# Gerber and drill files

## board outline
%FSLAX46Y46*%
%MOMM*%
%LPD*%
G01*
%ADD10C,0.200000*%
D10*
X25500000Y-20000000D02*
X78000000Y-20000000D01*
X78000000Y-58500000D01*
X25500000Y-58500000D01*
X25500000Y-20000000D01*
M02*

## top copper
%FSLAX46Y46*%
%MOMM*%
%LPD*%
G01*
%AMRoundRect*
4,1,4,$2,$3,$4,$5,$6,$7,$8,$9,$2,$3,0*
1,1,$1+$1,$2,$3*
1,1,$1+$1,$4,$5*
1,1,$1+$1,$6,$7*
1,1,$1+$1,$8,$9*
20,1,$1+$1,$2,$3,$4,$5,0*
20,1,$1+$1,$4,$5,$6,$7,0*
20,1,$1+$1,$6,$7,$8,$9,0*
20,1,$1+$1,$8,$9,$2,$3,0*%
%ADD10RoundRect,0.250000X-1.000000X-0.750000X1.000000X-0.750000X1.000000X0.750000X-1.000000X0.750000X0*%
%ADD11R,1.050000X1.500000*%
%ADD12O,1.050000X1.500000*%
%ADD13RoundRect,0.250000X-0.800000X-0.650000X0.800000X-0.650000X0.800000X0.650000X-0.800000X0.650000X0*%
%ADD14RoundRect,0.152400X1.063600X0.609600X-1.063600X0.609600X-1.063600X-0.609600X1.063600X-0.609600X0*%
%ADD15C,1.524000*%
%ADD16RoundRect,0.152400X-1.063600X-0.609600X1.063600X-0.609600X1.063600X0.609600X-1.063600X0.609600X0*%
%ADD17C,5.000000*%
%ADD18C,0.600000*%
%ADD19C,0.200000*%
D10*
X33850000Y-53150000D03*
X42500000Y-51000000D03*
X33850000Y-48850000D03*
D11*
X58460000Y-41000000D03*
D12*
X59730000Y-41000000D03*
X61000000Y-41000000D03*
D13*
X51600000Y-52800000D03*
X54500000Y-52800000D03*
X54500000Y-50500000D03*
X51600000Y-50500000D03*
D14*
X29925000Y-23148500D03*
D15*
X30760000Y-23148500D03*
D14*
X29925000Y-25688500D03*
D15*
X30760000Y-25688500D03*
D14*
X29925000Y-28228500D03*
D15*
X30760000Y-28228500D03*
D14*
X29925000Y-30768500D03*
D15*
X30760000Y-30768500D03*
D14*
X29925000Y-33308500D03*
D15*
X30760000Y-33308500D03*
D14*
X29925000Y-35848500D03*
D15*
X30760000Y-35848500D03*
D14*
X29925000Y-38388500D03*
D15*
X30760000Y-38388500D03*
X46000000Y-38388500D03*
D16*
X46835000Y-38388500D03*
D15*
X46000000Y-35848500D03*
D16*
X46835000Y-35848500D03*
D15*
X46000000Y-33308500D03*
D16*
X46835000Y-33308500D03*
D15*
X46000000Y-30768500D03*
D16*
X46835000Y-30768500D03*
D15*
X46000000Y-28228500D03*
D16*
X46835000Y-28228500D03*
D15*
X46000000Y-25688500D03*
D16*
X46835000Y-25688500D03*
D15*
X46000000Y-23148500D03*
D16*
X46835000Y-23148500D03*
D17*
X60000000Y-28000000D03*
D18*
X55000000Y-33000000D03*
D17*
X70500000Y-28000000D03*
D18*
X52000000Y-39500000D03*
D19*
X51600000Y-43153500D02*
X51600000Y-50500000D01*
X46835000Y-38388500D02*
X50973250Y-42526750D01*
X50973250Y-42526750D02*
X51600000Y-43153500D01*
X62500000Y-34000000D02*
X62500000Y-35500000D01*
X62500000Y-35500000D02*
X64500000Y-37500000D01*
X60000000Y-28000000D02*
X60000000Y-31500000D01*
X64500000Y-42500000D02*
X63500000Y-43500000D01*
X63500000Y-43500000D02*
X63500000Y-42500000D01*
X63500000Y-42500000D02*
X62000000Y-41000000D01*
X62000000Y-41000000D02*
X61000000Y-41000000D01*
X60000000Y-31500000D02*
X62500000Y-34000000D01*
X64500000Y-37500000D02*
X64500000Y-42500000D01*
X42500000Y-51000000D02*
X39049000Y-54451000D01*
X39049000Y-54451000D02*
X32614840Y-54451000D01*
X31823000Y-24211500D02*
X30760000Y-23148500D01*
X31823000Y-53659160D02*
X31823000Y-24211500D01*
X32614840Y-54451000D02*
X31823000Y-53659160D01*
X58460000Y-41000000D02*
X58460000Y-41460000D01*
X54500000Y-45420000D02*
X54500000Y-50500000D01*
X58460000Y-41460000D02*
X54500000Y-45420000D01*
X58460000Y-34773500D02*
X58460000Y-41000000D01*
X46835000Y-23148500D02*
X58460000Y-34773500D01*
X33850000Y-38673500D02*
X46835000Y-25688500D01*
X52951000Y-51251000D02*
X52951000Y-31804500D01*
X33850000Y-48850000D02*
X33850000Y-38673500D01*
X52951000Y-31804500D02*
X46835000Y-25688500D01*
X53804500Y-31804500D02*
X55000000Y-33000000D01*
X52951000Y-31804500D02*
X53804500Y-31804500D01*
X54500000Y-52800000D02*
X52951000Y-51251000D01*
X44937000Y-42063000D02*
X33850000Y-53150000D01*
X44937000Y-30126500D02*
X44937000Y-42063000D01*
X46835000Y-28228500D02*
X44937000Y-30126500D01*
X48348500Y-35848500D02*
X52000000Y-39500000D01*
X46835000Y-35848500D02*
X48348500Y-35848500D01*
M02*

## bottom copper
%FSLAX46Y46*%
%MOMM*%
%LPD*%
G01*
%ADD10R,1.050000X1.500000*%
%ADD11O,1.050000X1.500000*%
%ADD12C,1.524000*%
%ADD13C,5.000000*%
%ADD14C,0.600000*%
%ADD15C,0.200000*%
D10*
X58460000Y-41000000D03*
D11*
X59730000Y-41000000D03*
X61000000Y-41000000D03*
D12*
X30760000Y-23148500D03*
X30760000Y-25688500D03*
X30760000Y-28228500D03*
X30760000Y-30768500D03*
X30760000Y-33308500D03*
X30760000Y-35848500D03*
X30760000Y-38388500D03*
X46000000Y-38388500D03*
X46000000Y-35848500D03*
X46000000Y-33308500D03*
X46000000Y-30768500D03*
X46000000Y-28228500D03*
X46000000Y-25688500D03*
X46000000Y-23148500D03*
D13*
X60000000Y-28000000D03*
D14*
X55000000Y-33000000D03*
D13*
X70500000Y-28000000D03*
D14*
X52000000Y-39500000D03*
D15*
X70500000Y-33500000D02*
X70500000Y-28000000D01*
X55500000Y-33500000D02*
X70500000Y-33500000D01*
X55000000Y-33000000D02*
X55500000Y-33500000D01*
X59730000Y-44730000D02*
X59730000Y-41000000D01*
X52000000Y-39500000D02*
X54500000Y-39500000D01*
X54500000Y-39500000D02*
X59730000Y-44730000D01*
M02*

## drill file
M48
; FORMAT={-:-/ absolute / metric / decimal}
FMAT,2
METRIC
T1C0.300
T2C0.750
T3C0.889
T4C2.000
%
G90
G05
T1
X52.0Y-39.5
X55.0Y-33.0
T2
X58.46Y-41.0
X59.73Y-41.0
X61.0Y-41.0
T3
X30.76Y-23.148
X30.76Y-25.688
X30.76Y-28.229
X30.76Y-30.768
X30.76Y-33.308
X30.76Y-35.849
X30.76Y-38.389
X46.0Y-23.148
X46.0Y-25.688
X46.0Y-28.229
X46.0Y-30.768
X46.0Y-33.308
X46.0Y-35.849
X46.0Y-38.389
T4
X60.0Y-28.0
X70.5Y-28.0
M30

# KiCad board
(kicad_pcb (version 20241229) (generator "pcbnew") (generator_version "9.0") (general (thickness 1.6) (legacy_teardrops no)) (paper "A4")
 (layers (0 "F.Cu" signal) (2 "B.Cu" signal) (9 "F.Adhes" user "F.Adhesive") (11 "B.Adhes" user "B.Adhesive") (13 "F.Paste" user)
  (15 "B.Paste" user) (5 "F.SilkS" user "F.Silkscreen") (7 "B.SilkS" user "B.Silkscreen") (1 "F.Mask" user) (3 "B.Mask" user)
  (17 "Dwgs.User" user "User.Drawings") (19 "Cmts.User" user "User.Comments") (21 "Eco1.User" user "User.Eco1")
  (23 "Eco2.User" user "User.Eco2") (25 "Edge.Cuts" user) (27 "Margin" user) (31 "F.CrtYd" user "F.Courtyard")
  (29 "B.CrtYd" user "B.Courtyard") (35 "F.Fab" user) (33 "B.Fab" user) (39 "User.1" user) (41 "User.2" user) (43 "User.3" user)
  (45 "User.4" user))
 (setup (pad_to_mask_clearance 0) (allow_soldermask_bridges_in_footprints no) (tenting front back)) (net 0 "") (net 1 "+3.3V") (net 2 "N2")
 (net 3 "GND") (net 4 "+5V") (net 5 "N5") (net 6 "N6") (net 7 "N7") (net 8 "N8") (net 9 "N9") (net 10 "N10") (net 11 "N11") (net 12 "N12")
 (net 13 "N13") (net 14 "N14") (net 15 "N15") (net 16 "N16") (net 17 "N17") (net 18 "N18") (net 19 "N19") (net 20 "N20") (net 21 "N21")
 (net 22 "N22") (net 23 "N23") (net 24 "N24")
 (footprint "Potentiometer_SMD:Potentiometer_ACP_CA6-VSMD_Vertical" (layer "F.Cu") (at 38.175 51)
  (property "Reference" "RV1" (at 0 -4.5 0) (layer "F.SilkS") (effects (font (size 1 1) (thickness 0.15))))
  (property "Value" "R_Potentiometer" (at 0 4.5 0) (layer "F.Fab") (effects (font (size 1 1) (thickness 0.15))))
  (pad "1" smd roundrect (at -4.325 2.15) (size 2.5 2) (layers "F.Cu" "F.Mask" "F.Paste") (roundrect_rratio 0.125) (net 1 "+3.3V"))
  (pad "2" smd roundrect (at 4.325 0) (size 2.5 2) (layers "F.Cu" "F.Mask" "F.Paste") (roundrect_rratio 0.125) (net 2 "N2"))
  (pad "3" smd roundrect (at -4.325 -2.15) (size 2.5 2) (layers "F.Cu" "F.Mask" "F.Paste") (roundrect_rratio 0.125) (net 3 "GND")))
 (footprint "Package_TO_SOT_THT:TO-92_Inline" (layer "F.Cu") (at 58.46 41)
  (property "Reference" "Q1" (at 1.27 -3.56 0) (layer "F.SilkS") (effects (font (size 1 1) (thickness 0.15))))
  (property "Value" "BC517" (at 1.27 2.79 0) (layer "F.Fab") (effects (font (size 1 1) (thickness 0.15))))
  (pad "1" thru_hole rect (at 0 0) (size 1.05 1.5) (drill 0.75) (layers "*.Cu" "*.Mask") (remove_unused_layers no) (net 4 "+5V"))
  (pad "2" thru_hole oval (at 1.27 0) (size 1.05 1.5) (drill 0.75) (layers "*.Cu" "*.Mask") (remove_unused_layers no) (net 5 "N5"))
  (pad "3" thru_hole oval (at 2.54 0) (size 1.05 1.5) (drill 0.75) (layers "*.Cu" "*.Mask") (remove_unused_layers no) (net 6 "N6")))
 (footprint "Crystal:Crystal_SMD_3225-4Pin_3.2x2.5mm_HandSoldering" (layer "F.Cu") (at 53.05 51.65)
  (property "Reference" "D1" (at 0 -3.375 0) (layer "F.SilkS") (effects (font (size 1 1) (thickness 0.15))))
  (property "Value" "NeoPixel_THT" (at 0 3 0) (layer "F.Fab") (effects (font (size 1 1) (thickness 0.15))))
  (pad "1" smd roundrect (at -1.45 1.15) (size 2.1 1.8) (layers "F.Cu" "F.Mask" "F.Paste") (roundrect_rratio 0.138889) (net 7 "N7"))
  (pad "2" smd roundrect (at 1.45 1.15) (size 2.1 1.8) (layers "F.Cu" "F.Mask" "F.Paste") (roundrect_rratio 0.138889) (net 3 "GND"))
  (pad "3" smd roundrect (at 1.45 -1.15) (size 2.1 1.8) (layers "F.Cu" "F.Mask" "F.Paste") (roundrect_rratio 0.138889) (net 4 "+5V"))
  (pad "4" smd roundrect (at -1.45 -1.15) (size 2.1 1.8) (layers "F.Cu" "F.Mask" "F.Paste") (roundrect_rratio 0.138889) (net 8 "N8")))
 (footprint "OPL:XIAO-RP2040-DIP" (layer "F.Cu") (at 38.38 30.7685)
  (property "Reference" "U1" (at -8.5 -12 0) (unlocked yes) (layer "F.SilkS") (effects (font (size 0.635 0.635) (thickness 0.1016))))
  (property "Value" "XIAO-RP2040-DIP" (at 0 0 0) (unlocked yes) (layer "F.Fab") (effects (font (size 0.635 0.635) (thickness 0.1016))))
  (pad "1" smd roundrect (at -8.455 -7.62 180) (size 2.432 1.524) (layers "F.Cu" "F.Mask") (roundrect_rratio 0.1) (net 2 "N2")
   (thermal_bridge_angle 45))
  (pad "1" thru_hole circle (at -7.62 -7.62 180) (size 1.524 1.524) (drill 0.889) (layers "*.Cu" "*.Mask") (remove_unused_layers no)
   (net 2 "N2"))
  (pad "2" smd roundrect (at -8.455 -5.08 180) (size 2.432 1.524) (layers "F.Cu" "F.Mask") (roundrect_rratio 0.1) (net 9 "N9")
   (thermal_bridge_angle 45))
  (pad "2" thru_hole circle (at -7.62 -5.08 180) (size 1.524 1.524) (drill 0.889) (layers "*.Cu" "*.Mask") (remove_unused_layers no)
   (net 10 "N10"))
  (pad "3" smd roundrect (at -8.455 -2.54 180) (size 2.432 1.524) (layers "F.Cu" "F.Mask") (roundrect_rratio 0.1) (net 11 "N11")
   (thermal_bridge_angle 45))
  (pad "3" thru_hole circle (at -7.62 -2.54 180) (size 1.524 1.524) (drill 0.889) (layers "*.Cu" "*.Mask") (remove_unused_layers no)
   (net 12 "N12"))
  (pad "4" smd roundrect (at -8.455 0 180) (size 2.432 1.524) (layers "F.Cu" "F.Mask") (roundrect_rratio 0.1) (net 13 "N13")
   (thermal_bridge_angle 45))
  (pad "4" thru_hole circle (at -7.62 0 180) (size 1.524 1.524) (drill 0.889) (layers "*.Cu" "*.Mask") (remove_unused_layers no)
   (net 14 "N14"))
  (pad "5" smd roundrect (at -8.455 2.54 180) (size 2.432 1.524) (layers "F.Cu" "F.Mask") (roundrect_rratio 0.1) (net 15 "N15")
   (thermal_bridge_angle 45))
  (pad "5" thru_hole circle (at -7.62 2.54 180) (size 1.524 1.524) (drill 0.889) (layers "*.Cu" "*.Mask") (remove_unused_layers no)
   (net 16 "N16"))
  (pad "6" smd roundrect (at -8.455 5.08 180) (size 2.432 1.524) (layers "F.Cu" "F.Mask") (roundrect_rratio 0.1) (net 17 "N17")
   (thermal_bridge_angle 45))
  (pad "6" thru_hole circle (at -7.62 5.08 180) (size 1.524 1.524) (drill 0.889) (layers "*.Cu" "*.Mask") (remove_unused_layers no)
   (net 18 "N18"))
  (pad "7" smd roundrect (at -8.455 7.62 180) (size 2.432 1.524) (layers "F.Cu" "F.Mask") (roundrect_rratio 0.1) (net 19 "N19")
   (thermal_bridge_angle 45))
  (pad "7" thru_hole circle (at -7.62 7.62 180) (size 1.524 1.524) (drill 0.889) (layers "*.Cu" "*.Mask") (remove_unused_layers no)
   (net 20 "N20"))
  (pad "8" thru_hole circle (at 7.62 7.62) (size 1.524 1.524) (drill 0.889) (layers "*.Cu" "*.Mask") (remove_unused_layers no) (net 8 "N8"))
  (pad "8" smd roundrect (at 8.455 7.62) (size 2.432 1.524) (layers "F.Cu" "F.Mask") (roundrect_rratio 0.1) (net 8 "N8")
   (thermal_bridge_angle 45))
  (pad "9" thru_hole circle (at 7.62 5.08) (size 1.524 1.524) (drill 0.889) (layers "*.Cu" "*.Mask") (remove_unused_layers no) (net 5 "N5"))
  (pad "9" smd roundrect (at 8.455 5.08) (size 2.432 1.524) (layers "F.Cu" "F.Mask") (roundrect_rratio 0.1) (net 5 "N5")
   (thermal_bridge_angle 45))
  (pad "10" thru_hole circle (at 7.62 2.54) (size 1.524 1.524) (drill 0.889) (layers "*.Cu" "*.Mask") (remove_unused_layers no)
   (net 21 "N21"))
  (pad "10" smd roundrect (at 8.455 2.54) (size 2.432 1.524) (layers "F.Cu" "F.Mask") (roundrect_rratio 0.1) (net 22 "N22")
   (thermal_bridge_angle 45))
  (pad "11" thru_hole circle (at 7.62 0) (size 1.524 1.524) (drill 0.889) (layers "*.Cu" "*.Mask") (remove_unused_layers no) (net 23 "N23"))
  (pad "11" smd roundrect (at 8.455 0) (size 2.432 1.524) (layers "F.Cu" "F.Mask") (roundrect_rratio 0.1) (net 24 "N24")
   (thermal_bridge_angle 45))
  (pad "12" thru_hole circle (at 7.62 -2.54) (size 1.524 1.524) (drill 0.889) (layers "*.Cu" "*.Mask") (remove_unused_layers no)
   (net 1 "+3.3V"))
  (pad "12" smd roundrect (at 8.455 -2.54) (size 2.432 1.524) (layers "F.Cu" "F.Mask") (roundrect_rratio 0.1) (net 1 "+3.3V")
   (thermal_bridge_angle 45))
  (pad "13" thru_hole circle (at 7.62 -5.08) (size 1.524 1.524) (drill 0.889) (layers "*.Cu" "*.Mask") (remove_unused_layers no)
   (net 3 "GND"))
  (pad "13" smd roundrect (at 8.455 -5.08) (size 2.432 1.524) (layers "F.Cu" "F.Mask") (roundrect_rratio 0.1) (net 3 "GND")
   (thermal_bridge_angle 45))
  (pad "14" thru_hole circle (at 7.62 -7.62) (size 1.524 1.524) (drill 0.889) (layers "*.Cu" "*.Mask") (remove_unused_layers no)
   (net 4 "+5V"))
  (pad "14" smd roundrect (at 8.455 -7.62) (size 2.432 1.524) (layers "F.Cu" "F.Mask") (roundrect_rratio 0.1) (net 4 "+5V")
   (thermal_bridge_angle 45)))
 (gr_rect (start 25.5 20) (end 78 58.5) (stroke (width 0.2) (type solid)) (fill no) (layer "Edge.Cuts"))
 (segment (start 51.6 43.1535) (end 51.6 50.5) (width 0.2) (layer "F.Cu") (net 8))
 (segment (start 46.835 38.3885) (end 50.97325 42.52675) (width 0.2) (layer "F.Cu") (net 8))
 (segment (start 50.97325 42.52675) (end 51.6 43.1535) (width 0.2) (layer "F.Cu") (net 8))
 (segment (start 62.5 34) (end 62.5 35.5) (width 0.2) (layer "F.Cu") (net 6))
 (segment (start 62.5 35.5) (end 64.5 37.5) (width 0.2) (layer "F.Cu") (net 6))
 (segment (start 60 28) (end 60 31.5) (width 0.2) (layer "F.Cu") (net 6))
 (segment (start 64.5 42.5) (end 63.5 43.5) (width 0.2) (layer "F.Cu") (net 6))
 (segment (start 63.5 43.5) (end 63.5 42.5) (width 0.2) (layer "F.Cu") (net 6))
 (segment (start 63.5 42.5) (end 62 41) (width 0.2) (layer "F.Cu") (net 6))
 (segment (start 62 41) (end 61 41) (width 0.2) (layer "F.Cu") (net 6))
 (segment (start 60 31.5) (end 62.5 34) (width 0.2) (layer "F.Cu") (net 6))
 (segment (start 64.5 37.5) (end 64.5 42.5) (width 0.2) (layer "F.Cu") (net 6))
 (via (at 60 28) (size 5) (drill 2) (layers "F.Cu" "B.Cu") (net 6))
 (segment (start 42.5 51) (end 39.049 54.451) (width 0.2) (layer "F.Cu") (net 2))
 (segment (start 39.049 54.451) (end 32.61484 54.451) (width 0.2) (layer "F.Cu") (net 2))
 (segment (start 31.823 24.2115) (end 30.76 23.1485) (width 0.2) (layer "F.Cu") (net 2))
 (segment (start 31.823 53.65916) (end 31.823 24.2115) (width 0.2) (layer "F.Cu") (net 2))
 (segment (start 32.61484 54.451) (end 31.823 53.65916) (width 0.2) (layer "F.Cu") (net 2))
 (segment (start 58.46 41) (end 58.46 41.46) (width 0.2) (layer "F.Cu") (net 4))
 (segment (start 54.5 45.42) (end 54.5 50.5) (width 0.2) (layer "F.Cu") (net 4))
 (segment (start 58.46 41.46) (end 54.5 45.42) (width 0.2) (layer "F.Cu") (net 4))
 (segment (start 58.46 34.7735) (end 58.46 41) (width 0.2) (layer "F.Cu") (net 4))
 (segment (start 46.835 23.1485) (end 58.46 34.7735) (width 0.2) (layer "F.Cu") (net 4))
 (segment (start 33.85 38.6735) (end 46.835 25.6885) (width 0.2) (layer "F.Cu") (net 3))
 (segment (start 52.951 51.251) (end 52.951 31.8045) (width 0.2) (layer "F.Cu") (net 3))
 (segment (start 33.85 48.85) (end 33.85 38.6735) (width 0.2) (layer "F.Cu") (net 3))
 (segment (start 52.951 31.8045) (end 46.835 25.6885) (width 0.2) (layer "F.Cu") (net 3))
 (segment (start 53.8045 31.8045) (end 55 33) (width 0.2) (layer "F.Cu") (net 3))
 (segment (start 52.951 31.8045) (end 53.8045 31.8045) (width 0.2) (layer "F.Cu") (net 3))
 (segment (start 54.5 52.8) (end 52.951 51.251) (width 0.2) (layer "F.Cu") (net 3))
 (via (at 55 33) (size 0.6) (drill 0.3) (layers "F.Cu" "B.Cu") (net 3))
 (via (at 70.5 28) (size 5) (drill 2) (layers "F.Cu" "B.Cu") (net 3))
 (segment (start 70.5 33.5) (end 70.5 28) (width 0.2) (layer "B.Cu") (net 3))
 (segment (start 55.5 33.5) (end 70.5 33.5) (width 0.2) (layer "B.Cu") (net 3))
 (segment (start 55 33) (end 55.5 33.5) (width 0.2) (layer "B.Cu") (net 3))
 (segment (start 44.937 42.063) (end 33.85 53.15) (width 0.2) (layer "F.Cu") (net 1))
 (segment (start 44.937 30.1265) (end 44.937 42.063) (width 0.2) (layer "F.Cu") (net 1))
 (segment (start 46.835 28.2285) (end 44.937 30.1265) (width 0.2) (layer "F.Cu") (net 1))
 (segment (start 48.3485 35.8485) (end 52 39.5) (width 0.2) (layer "F.Cu") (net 5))
 (segment (start 46.835 35.8485) (end 48.3485 35.8485) (width 0.2) (layer "F.Cu") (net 5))
 (via (at 52 39.5) (size 0.6) (drill 0.3) (layers "F.Cu" "B.Cu") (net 5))
 (segment (start 59.73 44.73) (end 59.73 41) (width 0.2) (layer "B.Cu") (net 5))
 (segment (start 52 39.5) (end 54.5 39.5) (width 0.2) (layer "B.Cu") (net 5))
 (segment (start 54.5 39.5) (end 59.73 44.73) (width 0.2) (layer "B.Cu") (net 5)))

